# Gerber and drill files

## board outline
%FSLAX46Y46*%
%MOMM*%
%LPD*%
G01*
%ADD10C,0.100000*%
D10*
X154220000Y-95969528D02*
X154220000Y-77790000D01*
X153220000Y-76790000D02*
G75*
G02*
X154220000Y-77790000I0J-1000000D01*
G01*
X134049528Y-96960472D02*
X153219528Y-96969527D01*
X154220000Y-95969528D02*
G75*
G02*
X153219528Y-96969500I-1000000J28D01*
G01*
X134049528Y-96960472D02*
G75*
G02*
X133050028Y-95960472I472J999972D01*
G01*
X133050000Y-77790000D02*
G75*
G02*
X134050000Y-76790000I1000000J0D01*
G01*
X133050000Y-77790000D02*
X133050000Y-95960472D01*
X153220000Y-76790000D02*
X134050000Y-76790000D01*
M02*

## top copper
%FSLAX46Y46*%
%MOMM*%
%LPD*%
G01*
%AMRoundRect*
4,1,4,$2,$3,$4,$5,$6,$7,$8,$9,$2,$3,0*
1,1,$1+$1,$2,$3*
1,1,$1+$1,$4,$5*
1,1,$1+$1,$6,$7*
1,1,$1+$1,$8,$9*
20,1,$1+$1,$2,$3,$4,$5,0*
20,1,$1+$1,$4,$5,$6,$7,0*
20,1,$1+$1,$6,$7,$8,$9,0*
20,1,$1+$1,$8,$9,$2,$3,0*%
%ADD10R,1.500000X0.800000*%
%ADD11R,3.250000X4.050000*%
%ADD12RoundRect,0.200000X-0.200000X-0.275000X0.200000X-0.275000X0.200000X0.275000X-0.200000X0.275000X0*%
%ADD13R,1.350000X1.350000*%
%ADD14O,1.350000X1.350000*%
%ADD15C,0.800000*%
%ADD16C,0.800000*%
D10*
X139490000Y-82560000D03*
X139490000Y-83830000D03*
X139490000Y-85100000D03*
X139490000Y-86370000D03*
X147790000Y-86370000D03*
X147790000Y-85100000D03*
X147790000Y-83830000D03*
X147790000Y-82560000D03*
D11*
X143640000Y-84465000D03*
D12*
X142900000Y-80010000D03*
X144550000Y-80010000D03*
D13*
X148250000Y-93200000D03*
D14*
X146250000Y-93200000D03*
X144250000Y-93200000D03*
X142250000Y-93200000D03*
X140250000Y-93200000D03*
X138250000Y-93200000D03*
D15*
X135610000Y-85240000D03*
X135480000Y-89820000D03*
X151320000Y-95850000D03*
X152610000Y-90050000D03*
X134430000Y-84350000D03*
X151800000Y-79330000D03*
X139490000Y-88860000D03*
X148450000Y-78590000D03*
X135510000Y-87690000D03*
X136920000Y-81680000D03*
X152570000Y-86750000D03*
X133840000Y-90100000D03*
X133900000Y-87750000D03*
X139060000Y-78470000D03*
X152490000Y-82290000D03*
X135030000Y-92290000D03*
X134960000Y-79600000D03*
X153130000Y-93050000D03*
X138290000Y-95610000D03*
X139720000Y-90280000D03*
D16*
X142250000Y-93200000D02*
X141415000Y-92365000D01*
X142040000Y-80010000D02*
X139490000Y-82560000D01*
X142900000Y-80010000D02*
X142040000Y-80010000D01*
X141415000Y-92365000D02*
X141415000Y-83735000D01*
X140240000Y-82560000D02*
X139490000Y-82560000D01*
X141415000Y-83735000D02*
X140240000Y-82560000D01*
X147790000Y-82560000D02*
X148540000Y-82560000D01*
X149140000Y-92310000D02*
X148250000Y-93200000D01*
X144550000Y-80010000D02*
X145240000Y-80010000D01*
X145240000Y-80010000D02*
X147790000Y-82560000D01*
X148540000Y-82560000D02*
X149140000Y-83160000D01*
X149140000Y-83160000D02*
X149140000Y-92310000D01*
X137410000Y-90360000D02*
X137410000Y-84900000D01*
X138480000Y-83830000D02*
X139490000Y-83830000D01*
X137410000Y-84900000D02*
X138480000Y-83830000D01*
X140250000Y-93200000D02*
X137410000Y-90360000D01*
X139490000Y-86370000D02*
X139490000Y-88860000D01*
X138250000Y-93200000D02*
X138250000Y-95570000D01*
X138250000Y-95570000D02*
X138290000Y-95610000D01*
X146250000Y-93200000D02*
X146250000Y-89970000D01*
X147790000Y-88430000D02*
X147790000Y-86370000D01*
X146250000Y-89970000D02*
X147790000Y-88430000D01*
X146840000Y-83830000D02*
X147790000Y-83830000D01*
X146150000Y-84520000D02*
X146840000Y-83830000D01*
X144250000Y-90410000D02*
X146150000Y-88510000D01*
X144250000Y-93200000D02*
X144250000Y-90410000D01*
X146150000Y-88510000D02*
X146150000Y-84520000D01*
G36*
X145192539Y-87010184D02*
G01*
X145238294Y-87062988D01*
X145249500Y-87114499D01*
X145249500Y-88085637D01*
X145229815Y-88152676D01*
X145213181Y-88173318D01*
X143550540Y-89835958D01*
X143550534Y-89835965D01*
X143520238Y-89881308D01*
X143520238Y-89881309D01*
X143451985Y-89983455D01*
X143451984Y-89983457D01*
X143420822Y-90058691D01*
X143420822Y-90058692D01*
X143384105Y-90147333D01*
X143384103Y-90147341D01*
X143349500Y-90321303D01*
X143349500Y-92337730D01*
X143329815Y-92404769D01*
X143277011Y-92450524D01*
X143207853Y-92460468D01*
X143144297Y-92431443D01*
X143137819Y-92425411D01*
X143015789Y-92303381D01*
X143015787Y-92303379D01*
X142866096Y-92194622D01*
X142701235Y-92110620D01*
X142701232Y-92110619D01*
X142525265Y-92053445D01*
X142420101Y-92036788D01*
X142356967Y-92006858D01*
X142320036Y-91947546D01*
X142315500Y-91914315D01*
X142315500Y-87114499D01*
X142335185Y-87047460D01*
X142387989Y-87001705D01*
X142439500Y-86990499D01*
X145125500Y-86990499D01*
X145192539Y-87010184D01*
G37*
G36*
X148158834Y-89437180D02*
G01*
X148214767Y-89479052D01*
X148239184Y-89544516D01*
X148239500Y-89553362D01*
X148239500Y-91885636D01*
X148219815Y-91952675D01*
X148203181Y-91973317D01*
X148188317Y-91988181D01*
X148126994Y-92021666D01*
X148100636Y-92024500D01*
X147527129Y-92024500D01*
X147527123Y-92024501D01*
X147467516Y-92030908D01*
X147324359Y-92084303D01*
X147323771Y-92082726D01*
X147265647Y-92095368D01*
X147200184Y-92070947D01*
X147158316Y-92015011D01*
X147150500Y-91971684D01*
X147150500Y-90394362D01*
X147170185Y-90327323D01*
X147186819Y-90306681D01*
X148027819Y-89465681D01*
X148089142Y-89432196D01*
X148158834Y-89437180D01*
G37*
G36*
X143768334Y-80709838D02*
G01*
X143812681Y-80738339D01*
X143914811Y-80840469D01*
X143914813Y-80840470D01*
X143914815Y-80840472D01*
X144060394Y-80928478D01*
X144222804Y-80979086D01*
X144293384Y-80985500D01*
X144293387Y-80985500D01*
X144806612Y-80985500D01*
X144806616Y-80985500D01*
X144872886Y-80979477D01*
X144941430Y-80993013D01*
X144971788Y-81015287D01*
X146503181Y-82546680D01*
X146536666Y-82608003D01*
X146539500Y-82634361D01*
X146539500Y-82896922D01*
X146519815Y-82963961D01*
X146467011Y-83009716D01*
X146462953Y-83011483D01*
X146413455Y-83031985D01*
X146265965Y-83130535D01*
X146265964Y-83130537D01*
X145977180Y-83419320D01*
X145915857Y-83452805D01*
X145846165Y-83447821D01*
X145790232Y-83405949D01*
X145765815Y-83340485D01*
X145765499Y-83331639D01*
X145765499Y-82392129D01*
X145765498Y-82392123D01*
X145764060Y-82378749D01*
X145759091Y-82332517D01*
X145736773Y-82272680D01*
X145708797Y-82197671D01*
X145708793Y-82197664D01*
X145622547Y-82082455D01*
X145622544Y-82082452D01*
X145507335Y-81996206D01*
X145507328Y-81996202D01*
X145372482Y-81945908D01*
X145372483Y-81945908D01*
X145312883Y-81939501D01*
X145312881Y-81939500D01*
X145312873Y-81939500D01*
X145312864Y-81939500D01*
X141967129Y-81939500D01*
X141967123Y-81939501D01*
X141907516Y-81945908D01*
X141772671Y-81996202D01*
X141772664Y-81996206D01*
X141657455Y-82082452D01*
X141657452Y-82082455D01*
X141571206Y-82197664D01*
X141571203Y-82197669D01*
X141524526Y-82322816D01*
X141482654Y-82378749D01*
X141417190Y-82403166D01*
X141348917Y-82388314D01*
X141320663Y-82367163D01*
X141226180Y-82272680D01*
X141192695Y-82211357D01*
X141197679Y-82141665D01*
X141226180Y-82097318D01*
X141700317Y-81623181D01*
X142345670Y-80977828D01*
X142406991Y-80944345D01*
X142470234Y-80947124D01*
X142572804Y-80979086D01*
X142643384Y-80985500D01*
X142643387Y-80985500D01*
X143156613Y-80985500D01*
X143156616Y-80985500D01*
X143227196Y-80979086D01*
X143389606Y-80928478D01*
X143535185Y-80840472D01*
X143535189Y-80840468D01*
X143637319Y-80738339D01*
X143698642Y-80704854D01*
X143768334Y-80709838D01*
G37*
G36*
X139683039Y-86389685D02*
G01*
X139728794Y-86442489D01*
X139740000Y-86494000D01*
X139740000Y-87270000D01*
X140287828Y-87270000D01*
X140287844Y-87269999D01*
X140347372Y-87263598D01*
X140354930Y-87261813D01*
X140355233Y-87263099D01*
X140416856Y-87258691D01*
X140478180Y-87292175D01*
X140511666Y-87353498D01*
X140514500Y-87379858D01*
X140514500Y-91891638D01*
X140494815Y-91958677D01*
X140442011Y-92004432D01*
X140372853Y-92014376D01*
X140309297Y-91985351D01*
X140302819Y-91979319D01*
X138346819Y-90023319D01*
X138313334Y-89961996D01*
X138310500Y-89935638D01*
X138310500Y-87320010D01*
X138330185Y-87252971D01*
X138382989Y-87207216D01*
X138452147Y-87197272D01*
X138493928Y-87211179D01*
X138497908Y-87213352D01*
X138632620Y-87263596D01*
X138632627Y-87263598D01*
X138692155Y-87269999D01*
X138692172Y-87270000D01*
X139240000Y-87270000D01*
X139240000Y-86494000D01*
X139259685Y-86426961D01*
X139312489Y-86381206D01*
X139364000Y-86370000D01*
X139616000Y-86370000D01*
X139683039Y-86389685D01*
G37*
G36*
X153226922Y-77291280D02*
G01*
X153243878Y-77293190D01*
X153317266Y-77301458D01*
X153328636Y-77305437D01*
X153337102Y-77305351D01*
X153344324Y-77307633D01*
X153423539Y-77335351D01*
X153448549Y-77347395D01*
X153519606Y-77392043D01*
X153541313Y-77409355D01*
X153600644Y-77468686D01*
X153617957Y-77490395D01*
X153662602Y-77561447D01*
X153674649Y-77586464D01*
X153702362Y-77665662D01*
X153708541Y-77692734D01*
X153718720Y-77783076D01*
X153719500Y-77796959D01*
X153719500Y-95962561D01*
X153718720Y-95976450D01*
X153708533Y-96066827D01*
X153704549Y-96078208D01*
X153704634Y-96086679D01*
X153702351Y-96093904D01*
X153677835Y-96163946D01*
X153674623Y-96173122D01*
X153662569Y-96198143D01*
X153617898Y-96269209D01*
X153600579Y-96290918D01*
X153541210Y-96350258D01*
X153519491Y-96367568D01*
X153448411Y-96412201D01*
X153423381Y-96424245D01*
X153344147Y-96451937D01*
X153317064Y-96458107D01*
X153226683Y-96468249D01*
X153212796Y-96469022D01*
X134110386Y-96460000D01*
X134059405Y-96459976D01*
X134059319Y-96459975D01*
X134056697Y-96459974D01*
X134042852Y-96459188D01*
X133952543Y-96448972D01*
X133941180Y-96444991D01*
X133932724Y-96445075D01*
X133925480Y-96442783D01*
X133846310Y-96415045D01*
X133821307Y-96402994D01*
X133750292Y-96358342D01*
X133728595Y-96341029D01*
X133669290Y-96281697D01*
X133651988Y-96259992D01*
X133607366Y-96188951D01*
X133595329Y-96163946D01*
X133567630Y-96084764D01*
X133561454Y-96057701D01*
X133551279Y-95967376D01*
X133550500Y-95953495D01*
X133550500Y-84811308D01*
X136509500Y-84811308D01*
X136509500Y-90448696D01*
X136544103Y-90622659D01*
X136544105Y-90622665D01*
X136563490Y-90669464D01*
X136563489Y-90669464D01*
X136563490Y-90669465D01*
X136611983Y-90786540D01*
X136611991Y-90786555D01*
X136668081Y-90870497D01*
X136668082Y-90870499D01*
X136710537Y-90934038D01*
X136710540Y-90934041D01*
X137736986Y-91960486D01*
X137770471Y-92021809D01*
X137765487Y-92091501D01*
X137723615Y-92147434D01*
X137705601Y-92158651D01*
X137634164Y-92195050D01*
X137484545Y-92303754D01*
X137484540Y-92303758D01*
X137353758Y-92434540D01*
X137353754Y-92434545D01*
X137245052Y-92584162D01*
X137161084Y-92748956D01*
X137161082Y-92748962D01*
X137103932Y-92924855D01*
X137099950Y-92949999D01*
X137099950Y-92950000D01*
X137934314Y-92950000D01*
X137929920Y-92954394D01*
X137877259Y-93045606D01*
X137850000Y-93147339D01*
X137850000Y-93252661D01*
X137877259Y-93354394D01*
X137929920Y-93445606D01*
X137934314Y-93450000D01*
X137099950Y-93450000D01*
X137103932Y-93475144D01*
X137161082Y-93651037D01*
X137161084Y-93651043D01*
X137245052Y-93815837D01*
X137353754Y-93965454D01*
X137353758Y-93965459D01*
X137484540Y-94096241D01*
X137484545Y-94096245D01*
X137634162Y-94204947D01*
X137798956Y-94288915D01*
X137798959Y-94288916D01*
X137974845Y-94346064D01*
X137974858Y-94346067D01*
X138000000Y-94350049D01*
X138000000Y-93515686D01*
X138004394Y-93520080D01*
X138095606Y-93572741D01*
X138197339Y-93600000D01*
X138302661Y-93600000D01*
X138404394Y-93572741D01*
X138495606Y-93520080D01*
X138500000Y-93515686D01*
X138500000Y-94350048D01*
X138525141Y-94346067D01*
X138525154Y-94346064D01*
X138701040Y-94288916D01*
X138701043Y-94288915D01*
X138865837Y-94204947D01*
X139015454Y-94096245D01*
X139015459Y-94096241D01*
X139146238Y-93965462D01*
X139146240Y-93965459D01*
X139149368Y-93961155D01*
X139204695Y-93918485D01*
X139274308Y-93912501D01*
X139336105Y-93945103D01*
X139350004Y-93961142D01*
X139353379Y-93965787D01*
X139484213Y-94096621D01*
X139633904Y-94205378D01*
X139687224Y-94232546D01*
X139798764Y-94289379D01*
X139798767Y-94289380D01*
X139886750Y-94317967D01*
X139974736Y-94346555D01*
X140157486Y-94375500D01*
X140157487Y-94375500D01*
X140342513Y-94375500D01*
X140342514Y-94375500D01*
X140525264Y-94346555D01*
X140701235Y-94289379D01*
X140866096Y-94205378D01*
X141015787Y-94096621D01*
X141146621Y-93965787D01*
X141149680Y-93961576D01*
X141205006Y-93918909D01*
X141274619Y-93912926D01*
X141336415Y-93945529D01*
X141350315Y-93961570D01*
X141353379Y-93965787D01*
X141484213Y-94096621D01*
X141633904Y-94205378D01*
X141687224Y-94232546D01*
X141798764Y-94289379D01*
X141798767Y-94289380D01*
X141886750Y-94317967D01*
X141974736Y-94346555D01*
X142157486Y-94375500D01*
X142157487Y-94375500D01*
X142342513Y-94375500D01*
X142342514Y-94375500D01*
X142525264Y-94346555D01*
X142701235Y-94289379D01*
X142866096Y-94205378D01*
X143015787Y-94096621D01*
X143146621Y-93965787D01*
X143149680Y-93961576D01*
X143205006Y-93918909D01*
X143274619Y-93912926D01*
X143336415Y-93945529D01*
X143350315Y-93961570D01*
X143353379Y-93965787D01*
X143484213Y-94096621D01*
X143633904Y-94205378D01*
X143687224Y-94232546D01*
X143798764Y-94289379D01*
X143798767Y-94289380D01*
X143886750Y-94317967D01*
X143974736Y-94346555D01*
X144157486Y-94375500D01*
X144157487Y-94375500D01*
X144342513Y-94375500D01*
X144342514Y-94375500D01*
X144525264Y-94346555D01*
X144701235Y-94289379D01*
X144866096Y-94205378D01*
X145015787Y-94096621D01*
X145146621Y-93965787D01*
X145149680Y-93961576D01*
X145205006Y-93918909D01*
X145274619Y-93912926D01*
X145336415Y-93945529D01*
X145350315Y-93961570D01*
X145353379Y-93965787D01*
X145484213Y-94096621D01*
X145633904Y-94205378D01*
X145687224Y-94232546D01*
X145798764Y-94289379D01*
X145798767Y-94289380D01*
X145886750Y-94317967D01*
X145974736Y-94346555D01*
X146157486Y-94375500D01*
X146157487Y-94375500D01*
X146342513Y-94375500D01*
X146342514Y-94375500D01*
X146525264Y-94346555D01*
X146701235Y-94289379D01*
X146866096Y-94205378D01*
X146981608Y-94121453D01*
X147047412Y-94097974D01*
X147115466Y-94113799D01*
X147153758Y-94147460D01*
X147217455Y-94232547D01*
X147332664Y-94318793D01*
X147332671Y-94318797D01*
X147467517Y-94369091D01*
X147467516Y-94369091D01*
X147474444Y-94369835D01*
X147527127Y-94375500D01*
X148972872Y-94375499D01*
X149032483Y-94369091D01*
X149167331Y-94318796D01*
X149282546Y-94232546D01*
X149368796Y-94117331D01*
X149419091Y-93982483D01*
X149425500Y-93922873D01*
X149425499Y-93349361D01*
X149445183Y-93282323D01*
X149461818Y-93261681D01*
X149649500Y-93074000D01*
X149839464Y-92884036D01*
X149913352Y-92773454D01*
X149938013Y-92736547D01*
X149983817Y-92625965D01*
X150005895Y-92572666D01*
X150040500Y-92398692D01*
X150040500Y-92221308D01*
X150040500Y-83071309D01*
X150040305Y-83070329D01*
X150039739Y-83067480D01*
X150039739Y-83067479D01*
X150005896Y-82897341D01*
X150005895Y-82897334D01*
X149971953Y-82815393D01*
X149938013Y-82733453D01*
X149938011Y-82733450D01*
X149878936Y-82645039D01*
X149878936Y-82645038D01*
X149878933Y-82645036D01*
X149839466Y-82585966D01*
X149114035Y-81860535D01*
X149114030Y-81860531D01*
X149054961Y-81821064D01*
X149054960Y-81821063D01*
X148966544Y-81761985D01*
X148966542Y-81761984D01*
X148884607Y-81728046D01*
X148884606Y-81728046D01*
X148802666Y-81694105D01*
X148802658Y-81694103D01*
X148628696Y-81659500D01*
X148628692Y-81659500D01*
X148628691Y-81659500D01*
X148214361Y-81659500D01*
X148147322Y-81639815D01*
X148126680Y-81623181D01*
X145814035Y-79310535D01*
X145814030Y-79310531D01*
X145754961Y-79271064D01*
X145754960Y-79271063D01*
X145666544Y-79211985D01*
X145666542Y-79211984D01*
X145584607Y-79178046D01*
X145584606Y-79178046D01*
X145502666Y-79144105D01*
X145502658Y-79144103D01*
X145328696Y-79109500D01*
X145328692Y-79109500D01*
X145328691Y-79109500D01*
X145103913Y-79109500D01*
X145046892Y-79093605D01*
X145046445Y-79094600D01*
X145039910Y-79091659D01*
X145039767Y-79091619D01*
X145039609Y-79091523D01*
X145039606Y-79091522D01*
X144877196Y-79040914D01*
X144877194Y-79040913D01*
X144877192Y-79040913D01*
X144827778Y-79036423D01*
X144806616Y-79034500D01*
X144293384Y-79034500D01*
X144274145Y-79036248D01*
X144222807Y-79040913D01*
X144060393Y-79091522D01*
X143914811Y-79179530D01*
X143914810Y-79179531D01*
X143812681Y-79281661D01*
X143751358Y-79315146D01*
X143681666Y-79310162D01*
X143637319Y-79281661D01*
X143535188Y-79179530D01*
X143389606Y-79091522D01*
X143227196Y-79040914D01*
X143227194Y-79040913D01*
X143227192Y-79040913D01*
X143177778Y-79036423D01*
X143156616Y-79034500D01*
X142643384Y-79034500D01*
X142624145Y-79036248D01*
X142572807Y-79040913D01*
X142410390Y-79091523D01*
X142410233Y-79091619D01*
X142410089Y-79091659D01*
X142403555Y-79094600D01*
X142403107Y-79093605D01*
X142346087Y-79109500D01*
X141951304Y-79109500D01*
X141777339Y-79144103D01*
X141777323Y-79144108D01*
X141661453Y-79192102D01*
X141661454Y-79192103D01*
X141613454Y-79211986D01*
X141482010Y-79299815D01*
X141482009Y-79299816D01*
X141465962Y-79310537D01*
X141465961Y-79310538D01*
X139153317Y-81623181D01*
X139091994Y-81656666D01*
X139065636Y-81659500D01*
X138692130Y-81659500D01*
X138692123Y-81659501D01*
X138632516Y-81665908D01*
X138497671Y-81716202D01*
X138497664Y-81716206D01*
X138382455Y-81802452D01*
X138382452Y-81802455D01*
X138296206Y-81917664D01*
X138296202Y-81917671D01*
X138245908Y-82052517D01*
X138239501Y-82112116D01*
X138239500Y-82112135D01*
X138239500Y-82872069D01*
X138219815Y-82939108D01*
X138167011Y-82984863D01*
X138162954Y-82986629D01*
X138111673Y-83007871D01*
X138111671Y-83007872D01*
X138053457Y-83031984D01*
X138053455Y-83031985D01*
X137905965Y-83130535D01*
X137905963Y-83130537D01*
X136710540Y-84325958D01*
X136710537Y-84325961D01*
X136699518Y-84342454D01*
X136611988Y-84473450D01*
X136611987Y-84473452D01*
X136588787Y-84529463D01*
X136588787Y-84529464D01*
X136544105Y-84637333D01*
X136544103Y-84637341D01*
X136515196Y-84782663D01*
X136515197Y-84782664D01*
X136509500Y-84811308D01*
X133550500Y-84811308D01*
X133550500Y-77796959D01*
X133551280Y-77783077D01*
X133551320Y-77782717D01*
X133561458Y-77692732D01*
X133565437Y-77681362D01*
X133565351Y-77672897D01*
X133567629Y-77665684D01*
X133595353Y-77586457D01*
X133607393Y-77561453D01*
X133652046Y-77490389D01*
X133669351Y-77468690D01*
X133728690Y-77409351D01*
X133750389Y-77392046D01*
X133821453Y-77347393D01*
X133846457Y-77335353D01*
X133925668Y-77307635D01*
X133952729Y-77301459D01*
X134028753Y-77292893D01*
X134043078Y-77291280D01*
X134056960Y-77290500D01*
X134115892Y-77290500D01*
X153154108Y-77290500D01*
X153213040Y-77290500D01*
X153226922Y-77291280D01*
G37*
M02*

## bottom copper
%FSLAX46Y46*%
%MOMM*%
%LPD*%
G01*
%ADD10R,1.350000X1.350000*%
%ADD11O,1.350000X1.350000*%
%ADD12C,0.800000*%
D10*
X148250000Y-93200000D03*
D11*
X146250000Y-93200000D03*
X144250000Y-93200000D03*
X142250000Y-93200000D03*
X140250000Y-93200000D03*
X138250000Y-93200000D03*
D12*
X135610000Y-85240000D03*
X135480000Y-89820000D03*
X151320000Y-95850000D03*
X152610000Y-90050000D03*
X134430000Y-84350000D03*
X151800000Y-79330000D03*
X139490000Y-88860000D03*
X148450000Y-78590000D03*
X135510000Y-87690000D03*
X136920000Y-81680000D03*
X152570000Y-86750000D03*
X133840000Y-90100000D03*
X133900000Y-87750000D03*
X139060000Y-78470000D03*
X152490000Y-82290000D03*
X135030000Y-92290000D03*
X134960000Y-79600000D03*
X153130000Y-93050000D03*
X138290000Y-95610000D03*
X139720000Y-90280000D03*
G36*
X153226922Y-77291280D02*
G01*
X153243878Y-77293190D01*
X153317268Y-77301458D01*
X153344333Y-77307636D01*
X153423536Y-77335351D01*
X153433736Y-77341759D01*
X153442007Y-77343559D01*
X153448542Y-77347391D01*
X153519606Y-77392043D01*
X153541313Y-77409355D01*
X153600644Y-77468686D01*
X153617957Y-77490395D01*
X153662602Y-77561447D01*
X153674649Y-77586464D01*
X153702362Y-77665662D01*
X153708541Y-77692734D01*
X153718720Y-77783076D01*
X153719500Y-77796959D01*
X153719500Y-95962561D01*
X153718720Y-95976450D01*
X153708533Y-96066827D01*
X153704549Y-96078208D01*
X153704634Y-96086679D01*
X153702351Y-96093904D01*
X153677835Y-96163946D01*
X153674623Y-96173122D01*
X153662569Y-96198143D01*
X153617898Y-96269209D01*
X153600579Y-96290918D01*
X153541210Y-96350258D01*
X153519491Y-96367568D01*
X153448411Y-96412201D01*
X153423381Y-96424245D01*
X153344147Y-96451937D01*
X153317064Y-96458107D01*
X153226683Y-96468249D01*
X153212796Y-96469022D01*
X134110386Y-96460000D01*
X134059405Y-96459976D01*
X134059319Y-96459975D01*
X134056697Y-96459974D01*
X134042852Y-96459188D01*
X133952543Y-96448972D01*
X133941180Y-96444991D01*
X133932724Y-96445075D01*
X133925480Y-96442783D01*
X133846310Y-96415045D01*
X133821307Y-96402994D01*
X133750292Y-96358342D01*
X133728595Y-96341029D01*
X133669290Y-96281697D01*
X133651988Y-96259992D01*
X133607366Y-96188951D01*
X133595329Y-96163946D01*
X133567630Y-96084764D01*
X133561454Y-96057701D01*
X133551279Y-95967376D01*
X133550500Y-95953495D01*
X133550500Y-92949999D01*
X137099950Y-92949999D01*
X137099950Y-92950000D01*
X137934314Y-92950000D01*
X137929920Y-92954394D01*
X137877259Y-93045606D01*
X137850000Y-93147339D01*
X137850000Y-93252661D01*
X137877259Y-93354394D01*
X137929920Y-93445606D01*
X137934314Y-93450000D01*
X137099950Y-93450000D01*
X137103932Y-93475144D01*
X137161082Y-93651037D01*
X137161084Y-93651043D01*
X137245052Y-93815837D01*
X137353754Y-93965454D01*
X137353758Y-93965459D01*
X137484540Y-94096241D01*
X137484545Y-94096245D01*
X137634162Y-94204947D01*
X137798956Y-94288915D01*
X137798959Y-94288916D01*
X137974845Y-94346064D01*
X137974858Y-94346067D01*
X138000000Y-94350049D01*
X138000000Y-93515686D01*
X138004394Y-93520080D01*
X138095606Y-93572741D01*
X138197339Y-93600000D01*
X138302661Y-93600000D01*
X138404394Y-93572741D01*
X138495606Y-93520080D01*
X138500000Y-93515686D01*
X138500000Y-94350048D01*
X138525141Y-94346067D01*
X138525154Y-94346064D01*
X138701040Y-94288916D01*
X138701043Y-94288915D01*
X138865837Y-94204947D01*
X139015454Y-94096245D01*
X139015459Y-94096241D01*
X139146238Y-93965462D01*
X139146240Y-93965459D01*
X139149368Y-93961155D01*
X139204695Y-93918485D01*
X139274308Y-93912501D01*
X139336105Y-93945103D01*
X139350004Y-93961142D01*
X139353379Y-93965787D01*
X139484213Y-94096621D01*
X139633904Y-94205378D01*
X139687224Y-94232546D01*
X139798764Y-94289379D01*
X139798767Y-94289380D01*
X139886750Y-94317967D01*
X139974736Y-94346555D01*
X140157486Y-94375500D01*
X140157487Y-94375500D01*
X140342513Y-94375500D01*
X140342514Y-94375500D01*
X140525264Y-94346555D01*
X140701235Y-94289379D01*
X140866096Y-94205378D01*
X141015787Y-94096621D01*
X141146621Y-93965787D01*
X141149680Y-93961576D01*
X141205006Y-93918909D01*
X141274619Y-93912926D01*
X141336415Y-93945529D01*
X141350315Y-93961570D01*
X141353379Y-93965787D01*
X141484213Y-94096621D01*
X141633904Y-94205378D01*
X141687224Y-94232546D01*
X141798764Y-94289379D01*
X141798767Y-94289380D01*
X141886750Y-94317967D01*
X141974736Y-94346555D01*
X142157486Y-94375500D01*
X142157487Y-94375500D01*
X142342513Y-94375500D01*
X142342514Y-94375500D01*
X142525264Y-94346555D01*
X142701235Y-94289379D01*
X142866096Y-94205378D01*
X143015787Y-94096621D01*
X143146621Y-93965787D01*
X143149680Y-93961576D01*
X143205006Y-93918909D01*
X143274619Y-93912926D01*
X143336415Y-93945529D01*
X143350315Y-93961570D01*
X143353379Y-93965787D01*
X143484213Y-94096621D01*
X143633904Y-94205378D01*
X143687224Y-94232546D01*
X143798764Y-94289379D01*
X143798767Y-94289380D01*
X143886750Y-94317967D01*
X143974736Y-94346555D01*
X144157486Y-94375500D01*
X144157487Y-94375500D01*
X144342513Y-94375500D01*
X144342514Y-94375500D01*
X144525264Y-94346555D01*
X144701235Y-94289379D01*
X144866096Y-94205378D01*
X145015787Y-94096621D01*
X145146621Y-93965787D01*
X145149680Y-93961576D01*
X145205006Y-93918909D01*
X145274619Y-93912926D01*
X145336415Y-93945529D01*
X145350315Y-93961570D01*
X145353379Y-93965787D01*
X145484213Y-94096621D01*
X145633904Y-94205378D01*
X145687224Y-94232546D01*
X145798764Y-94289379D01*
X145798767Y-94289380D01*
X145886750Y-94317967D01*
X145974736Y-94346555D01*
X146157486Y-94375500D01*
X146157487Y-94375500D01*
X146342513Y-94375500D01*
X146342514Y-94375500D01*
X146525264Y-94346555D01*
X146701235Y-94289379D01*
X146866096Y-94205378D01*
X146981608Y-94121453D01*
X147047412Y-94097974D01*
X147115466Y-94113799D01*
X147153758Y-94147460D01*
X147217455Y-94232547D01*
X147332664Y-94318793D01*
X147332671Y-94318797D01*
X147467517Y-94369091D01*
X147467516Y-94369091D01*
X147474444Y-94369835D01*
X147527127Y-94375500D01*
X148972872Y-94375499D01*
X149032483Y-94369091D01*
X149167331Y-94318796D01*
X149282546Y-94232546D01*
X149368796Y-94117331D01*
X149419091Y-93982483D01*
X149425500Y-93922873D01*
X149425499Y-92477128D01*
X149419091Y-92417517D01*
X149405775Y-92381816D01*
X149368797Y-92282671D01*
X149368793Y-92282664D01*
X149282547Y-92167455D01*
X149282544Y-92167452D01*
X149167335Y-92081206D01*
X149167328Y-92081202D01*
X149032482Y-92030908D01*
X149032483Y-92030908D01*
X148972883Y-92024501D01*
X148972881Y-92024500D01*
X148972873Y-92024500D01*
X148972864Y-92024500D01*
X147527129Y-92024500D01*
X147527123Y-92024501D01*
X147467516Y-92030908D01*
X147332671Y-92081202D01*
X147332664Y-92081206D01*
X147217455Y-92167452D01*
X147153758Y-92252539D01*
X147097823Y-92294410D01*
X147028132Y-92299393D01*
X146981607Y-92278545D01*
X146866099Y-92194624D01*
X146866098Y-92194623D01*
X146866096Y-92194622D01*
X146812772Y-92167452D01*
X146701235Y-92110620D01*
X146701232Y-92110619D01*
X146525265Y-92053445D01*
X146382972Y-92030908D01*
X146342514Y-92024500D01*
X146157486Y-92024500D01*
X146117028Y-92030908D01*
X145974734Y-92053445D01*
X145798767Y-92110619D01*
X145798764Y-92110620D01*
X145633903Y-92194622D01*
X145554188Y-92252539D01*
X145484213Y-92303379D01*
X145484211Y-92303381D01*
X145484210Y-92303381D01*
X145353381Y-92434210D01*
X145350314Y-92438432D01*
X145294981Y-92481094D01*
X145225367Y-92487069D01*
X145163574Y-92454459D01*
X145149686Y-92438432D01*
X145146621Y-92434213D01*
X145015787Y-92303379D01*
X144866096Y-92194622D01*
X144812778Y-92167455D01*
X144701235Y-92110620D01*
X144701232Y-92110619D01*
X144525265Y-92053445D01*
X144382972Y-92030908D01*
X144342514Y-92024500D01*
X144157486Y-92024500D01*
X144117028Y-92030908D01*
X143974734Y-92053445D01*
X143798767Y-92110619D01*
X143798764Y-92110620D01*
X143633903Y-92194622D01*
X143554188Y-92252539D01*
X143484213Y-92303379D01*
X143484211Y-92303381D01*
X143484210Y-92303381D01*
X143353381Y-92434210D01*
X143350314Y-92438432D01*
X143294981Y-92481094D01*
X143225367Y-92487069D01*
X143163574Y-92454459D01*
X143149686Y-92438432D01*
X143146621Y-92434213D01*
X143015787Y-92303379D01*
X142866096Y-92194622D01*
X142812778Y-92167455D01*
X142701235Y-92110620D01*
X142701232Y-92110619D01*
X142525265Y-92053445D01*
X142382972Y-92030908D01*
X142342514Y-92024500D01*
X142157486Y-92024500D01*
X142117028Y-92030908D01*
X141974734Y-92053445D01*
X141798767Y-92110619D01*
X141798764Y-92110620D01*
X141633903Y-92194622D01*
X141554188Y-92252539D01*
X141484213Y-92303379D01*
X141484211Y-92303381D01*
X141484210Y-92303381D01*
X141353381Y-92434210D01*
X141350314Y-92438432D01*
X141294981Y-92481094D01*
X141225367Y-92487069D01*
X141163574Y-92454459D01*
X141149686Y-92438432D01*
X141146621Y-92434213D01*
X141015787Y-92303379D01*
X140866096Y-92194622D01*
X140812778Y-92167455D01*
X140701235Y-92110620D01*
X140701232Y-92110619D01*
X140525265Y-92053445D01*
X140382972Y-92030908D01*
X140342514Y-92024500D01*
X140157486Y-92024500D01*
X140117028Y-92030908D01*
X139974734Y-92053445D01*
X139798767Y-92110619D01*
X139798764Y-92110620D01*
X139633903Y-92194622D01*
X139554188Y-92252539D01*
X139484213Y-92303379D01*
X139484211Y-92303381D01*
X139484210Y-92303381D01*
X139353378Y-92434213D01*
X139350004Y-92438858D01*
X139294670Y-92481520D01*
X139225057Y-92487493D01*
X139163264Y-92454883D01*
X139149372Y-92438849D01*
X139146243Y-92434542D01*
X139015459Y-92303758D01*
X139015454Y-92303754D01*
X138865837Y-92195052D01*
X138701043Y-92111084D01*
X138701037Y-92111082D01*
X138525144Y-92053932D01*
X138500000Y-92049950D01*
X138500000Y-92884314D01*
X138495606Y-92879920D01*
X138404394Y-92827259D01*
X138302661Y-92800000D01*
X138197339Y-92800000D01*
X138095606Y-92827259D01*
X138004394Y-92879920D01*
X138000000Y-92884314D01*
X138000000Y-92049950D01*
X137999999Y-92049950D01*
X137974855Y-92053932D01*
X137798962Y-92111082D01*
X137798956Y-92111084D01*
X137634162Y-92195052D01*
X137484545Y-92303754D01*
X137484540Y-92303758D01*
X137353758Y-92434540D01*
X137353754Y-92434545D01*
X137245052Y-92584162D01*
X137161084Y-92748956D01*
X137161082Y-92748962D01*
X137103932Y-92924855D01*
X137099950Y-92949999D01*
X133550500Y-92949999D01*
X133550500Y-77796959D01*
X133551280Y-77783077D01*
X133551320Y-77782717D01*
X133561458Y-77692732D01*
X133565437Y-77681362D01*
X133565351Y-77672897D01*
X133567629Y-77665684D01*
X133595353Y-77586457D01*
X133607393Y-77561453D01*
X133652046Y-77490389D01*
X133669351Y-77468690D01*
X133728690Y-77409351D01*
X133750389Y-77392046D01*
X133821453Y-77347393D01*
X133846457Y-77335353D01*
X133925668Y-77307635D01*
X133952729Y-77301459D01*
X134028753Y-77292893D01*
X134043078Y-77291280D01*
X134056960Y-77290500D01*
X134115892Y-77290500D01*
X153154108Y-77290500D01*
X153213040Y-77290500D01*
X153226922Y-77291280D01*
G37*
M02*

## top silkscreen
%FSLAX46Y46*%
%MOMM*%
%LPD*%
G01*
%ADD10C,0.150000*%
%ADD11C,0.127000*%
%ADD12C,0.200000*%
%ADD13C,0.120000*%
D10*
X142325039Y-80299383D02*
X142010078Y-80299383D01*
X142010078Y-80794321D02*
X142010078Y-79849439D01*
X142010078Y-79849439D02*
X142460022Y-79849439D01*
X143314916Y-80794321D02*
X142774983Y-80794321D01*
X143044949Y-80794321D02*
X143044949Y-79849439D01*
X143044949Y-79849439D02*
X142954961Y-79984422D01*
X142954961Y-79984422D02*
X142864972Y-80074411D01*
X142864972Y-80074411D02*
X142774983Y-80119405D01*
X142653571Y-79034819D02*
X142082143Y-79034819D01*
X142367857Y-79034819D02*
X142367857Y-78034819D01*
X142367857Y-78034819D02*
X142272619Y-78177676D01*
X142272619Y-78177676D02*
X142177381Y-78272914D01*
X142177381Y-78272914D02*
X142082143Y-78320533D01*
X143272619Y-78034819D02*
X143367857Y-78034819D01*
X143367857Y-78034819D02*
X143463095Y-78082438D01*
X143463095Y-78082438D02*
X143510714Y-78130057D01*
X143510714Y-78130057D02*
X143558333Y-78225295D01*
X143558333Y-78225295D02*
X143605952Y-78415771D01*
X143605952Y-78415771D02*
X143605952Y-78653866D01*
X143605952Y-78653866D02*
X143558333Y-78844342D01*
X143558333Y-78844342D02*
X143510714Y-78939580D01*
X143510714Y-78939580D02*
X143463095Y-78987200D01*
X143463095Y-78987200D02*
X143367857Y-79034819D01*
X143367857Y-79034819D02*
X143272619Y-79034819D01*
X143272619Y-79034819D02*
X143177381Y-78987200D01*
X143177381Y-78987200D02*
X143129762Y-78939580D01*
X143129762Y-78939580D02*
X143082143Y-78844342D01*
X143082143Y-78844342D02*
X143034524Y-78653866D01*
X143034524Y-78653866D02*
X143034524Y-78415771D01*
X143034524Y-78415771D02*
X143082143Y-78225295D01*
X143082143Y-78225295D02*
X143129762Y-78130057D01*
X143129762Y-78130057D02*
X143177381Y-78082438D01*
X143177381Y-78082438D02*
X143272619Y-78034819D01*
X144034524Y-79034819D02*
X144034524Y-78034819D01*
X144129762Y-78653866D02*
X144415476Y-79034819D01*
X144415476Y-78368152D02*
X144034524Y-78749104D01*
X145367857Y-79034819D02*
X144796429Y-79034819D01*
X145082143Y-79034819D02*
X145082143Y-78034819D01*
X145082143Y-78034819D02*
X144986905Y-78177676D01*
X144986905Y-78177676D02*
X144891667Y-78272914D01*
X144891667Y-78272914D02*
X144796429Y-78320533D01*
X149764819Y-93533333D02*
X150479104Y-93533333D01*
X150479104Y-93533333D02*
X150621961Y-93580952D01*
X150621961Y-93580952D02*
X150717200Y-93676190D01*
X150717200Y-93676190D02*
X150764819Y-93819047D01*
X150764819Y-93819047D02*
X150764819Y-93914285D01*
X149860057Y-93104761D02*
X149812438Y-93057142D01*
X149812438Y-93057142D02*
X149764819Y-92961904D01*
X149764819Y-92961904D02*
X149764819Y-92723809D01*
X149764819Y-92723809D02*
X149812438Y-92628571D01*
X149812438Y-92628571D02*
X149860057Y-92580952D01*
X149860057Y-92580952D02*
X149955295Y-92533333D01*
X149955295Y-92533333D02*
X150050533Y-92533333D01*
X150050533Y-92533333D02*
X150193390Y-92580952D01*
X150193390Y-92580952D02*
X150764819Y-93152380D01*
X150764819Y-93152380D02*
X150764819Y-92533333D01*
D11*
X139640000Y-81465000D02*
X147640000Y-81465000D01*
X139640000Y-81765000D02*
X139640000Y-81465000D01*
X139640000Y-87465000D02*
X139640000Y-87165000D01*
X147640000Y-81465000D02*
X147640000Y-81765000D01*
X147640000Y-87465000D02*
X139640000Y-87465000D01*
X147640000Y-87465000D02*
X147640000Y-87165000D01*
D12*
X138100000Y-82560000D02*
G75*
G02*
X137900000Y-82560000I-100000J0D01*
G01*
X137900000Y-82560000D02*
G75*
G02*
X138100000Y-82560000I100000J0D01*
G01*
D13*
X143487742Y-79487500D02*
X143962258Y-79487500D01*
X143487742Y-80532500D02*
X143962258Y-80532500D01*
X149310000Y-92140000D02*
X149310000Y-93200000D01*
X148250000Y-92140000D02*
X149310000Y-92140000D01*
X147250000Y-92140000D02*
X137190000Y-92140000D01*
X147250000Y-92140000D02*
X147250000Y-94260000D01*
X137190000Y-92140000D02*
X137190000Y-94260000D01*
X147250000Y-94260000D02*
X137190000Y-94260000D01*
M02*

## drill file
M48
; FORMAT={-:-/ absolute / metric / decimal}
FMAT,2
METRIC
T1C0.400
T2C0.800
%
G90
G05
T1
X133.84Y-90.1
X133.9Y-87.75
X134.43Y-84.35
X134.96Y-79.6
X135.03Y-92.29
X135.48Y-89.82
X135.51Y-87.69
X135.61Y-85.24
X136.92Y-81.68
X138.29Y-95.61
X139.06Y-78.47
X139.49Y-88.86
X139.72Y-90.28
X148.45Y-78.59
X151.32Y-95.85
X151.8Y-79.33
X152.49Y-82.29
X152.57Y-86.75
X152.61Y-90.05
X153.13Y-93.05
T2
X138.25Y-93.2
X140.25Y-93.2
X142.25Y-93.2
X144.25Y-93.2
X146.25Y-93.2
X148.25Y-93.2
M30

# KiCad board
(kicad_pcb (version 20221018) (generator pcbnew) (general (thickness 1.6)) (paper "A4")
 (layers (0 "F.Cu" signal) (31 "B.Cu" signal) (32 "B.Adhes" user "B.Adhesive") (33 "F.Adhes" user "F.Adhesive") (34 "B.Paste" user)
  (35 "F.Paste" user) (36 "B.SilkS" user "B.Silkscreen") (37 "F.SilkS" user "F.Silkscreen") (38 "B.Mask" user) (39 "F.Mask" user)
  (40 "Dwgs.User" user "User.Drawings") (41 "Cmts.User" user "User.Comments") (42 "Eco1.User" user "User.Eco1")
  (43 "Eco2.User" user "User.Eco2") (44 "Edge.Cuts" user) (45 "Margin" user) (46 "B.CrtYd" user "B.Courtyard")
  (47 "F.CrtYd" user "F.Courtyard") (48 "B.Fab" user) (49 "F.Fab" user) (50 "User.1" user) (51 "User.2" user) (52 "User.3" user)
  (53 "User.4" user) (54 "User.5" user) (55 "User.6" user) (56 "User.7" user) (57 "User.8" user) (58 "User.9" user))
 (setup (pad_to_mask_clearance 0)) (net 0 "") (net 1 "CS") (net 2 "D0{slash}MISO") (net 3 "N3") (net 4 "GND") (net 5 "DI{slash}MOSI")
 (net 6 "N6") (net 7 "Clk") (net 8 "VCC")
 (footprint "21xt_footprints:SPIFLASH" (layer "F.Cu") (at 143.64 84.465)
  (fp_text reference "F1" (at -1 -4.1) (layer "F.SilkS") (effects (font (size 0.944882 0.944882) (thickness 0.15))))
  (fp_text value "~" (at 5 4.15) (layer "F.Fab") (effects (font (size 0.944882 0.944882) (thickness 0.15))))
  (fp_line (start -4 -3) (end 4 -3) (stroke (width 0.127) (type solid)) (layer "F.SilkS"))
  (fp_line (start -4 -2.7) (end -4 -3) (stroke (width 0.127) (type solid)) (layer "F.SilkS"))
  (fp_line (start -4 3) (end -4 2.7) (stroke (width 0.127) (type solid)) (layer "F.SilkS"))
  (fp_line (start 4 -3) (end 4 -2.7) (stroke (width 0.127) (type solid)) (layer "F.SilkS"))
  (fp_line (start 4 3) (end -4 3) (stroke (width 0.127) (type solid)) (layer "F.SilkS"))
  (fp_line (start 4 3) (end 4 2.7) (stroke (width 0.127) (type solid)) (layer "F.SilkS"))
  (fp_circle (center -5.64 -1.905) (end -5.54 -1.905) (stroke (width 0.2) (type solid)) (fill none) (layer "F.SilkS"))
  (pad "1" smd rect (at -4.15 -1.905) (size 1.5 0.8) (layers "F.Cu" "F.Mask") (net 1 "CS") (solder_mask_margin 0.102))
  (pad "2" smd rect (at -4.15 -0.635) (size 1.5 0.8) (layers "F.Cu" "F.Mask") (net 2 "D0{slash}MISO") (solder_mask_margin 0.102))
  (pad "3" smd rect (at -4.15 0.635) (size 1.5 0.8) (layers "F.Cu" "F.Mask") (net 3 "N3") (solder_mask_margin 0.102))
  (pad "4" smd rect (at -4.15 1.905) (size 1.5 0.8) (layers "F.Cu" "F.Mask") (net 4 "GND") (solder_mask_margin 0.102))
  (pad "5" smd rect (at 4.15 1.905) (size 1.5 0.8) (layers "F.Cu" "F.Mask") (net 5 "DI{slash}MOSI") (solder_mask_margin 0.102))
  (pad "6" smd rect (at 4.15 0.635) (size 1.5 0.8) (layers "F.Cu" "F.Mask") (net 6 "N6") (solder_mask_margin 0.102))
  (pad "7" smd rect (at 4.15 -0.635) (size 1.5 0.8) (layers "F.Cu" "F.Mask") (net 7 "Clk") (solder_mask_margin 0.102))
  (pad "8" smd rect (at 4.15 -1.905) (size 1.5 0.8) (layers "F.Cu" "F.Mask") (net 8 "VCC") (solder_mask_margin 0.102))
  (pad "9" smd rect (at 0 0) (size 3.25 4.05) (layers "F.Cu" "F.Mask") (solder_mask_margin 0.102)))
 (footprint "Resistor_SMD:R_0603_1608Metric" (layer "F.Cu") (at 143.725 80.01)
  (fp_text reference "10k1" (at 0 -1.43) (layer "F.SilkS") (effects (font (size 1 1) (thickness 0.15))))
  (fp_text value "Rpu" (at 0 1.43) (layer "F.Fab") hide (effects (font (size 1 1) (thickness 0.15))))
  (fp_line (start -0.237258 -0.5225) (end 0.237258 -0.5225) (stroke (width 0.12) (type solid)) (layer "F.SilkS"))
  (fp_line (start -0.237258 0.5225) (end 0.237258 0.5225) (stroke (width 0.12) (type solid)) (layer "F.SilkS"))
  (pad "1" smd roundrect (at -0.825 0) (size 0.8 0.95) (layers "F.Cu" "F.Paste" "F.Mask") (roundrect_rratio 0.25) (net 1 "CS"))
  (pad "2" smd roundrect (at 0.825 0) (size 0.8 0.95) (layers "F.Cu" "F.Paste" "F.Mask") (roundrect_rratio 0.25) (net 8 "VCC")))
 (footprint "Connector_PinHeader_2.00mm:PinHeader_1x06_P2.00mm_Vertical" (layer "F.Cu") (at 148.25 93.2 -90)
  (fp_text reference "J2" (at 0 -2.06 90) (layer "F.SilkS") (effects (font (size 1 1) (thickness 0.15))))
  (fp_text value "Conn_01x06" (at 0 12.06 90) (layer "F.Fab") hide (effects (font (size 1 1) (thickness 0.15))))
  (fp_line (start -1.06 -1.06) (end 0 -1.06) (stroke (width 0.12) (type solid)) (layer "F.SilkS"))
  (fp_line (start -1.06 0) (end -1.06 -1.06) (stroke (width 0.12) (type solid)) (layer "F.SilkS"))
  (fp_line (start -1.06 1) (end -1.06 11.06) (stroke (width 0.12) (type solid)) (layer "F.SilkS"))
  (fp_line (start -1.06 1) (end 1.06 1) (stroke (width 0.12) (type solid)) (layer "F.SilkS"))
  (fp_line (start -1.06 11.06) (end 1.06 11.06) (stroke (width 0.12) (type solid)) (layer "F.SilkS"))
  (fp_line (start 1.06 1) (end 1.06 11.06) (stroke (width 0.12) (type solid)) (layer "F.SilkS"))
  (pad "1" thru_hole rect (at 0 0 270) (size 1.35 1.35) (drill 0.8) (layers "*.Cu" "*.Mask") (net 8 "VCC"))
  (pad "2" thru_hole oval (at 0 2 270) (size 1.35 1.35) (drill 0.8) (layers "*.Cu" "*.Mask") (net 5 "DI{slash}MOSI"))
  (pad "3" thru_hole oval (at 0 4 270) (size 1.35 1.35) (drill 0.8) (layers "*.Cu" "*.Mask") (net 7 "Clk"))
  (pad "4" thru_hole oval (at 0 6 270) (size 1.35 1.35) (drill 0.8) (layers "*.Cu" "*.Mask") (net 1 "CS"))
  (pad "5" thru_hole oval (at 0 8 270) (size 1.35 1.35) (drill 0.8) (layers "*.Cu" "*.Mask") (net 2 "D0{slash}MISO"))
  (pad "6" thru_hole oval (at 0 10 270) (size 1.35 1.35) (drill 0.8) (layers "*.Cu" "*.Mask") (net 4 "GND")))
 (gr_line (start 154.22 95.969528) (end 154.22 77.79) (stroke (width 0.1) (type default)) (layer "Edge.Cuts"))
 (gr_arc (start 153.22 76.79) (mid 153.927107 77.082893) (end 154.22 77.79) (stroke (width 0.1) (type default)) (layer "Edge.Cuts"))
 (gr_line (start 134.049528 96.960472) (end 153.219528 96.969527) (stroke (width 0.1) (type default)) (layer "Edge.Cuts"))
 (gr_arc (start 154.22 95.969528) (mid 153.92694 96.676802) (end 153.219528 96.969527) (stroke (width 0.1) (type default))
  (layer "Edge.Cuts"))
 (gr_arc (start 134.049528 96.960472) (mid 133.342736 96.66741) (end 133.05 95.960472) (stroke (width 0.1) (type default))
  (layer "Edge.Cuts"))
 (gr_arc (start 133.05 77.79) (mid 133.342893 77.082893) (end 134.05 76.79) (stroke (width 0.1) (type default)) (layer "Edge.Cuts"))
 (gr_line (start 133.05 77.79) (end 133.05 95.960472) (stroke (width 0.1) (type default)) (layer "Edge.Cuts"))
 (gr_line (start 153.22 76.79) (end 134.05 76.79) (stroke (width 0.1) (type default)) (layer "Edge.Cuts"))
 (segment (start 142.25 93.2) (end 141.415 92.365) (width 0.8) (layer "F.Cu") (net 1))
 (segment (start 142.04 80.01) (end 139.49 82.56) (width 0.8) (layer "F.Cu") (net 1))
 (segment (start 142.9 80.01) (end 142.04 80.01) (width 0.8) (layer "F.Cu") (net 1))
 (segment (start 141.415 92.365) (end 141.415 83.735) (width 0.8) (layer "F.Cu") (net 1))
 (segment (start 140.24 82.56) (end 139.49 82.56) (width 0.8) (layer "F.Cu") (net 1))
 (segment (start 141.415 83.735) (end 140.24 82.56) (width 0.8) (layer "F.Cu") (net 1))
 (segment (start 147.79 82.56) (end 148.54 82.56) (width 0.8) (layer "F.Cu") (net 8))
 (segment (start 149.14 92.31) (end 148.25 93.2) (width 0.8) (layer "F.Cu") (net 8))
 (segment (start 144.55 80.01) (end 145.24 80.01) (width 0.8) (layer "F.Cu") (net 8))
 (segment (start 145.24 80.01) (end 147.79 82.56) (width 0.8) (layer "F.Cu") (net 8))
 (segment (start 148.54 82.56) (end 149.14 83.16) (width 0.8) (layer "F.Cu") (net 8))
 (segment (start 149.14 83.16) (end 149.14 92.31) (width 0.8) (layer "F.Cu") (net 8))
 (segment (start 137.41 90.36) (end 137.41 84.9) (width 0.8) (layer "F.Cu") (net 2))
 (segment (start 138.48 83.83) (end 139.49 83.83) (width 0.8) (layer "F.Cu") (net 2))
 (segment (start 137.41 84.9) (end 138.48 83.83) (width 0.8) (layer "F.Cu") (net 2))
 (segment (start 140.25 93.2) (end 137.41 90.36) (width 0.8) (layer "F.Cu") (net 2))
 (segment (start 139.49 86.37) (end 139.49 88.86) (width 0.8) (layer "F.Cu") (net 4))
 (segment (start 138.25 93.2) (end 138.25 95.57) (width 0.8) (layer "F.Cu") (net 4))
 (segment (start 138.25 95.57) (end 138.29 95.61) (width 0.8) (layer "F.Cu") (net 4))
 (via (at 135.61 85.24) (size 0.8) (drill 0.4) (layers "F.Cu" "B.Cu") (free) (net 4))
 (via (at 135.48 89.82) (size 0.8) (drill 0.4) (layers "F.Cu" "B.Cu") (free) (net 4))
 (via (at 151.32 95.85) (size 0.8) (drill 0.4) (layers "F.Cu" "B.Cu") (free) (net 4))
 (via (at 152.61 90.05) (size 0.8) (drill 0.4) (layers "F.Cu" "B.Cu") (free) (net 4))
 (via (at 134.43 84.35) (size 0.8) (drill 0.4) (layers "F.Cu" "B.Cu") (free) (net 4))
 (via (at 151.8 79.33) (size 0.8) (drill 0.4) (layers "F.Cu" "B.Cu") (free) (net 4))
 (via (at 139.49 88.86) (size 0.8) (drill 0.4) (layers "F.Cu" "B.Cu") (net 4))
 (via (at 148.45 78.59) (size 0.8) (drill 0.4) (layers "F.Cu" "B.Cu") (free) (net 4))
 (via (at 135.51 87.69) (size 0.8) (drill 0.4) (layers "F.Cu" "B.Cu") (free) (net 4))
 (via (at 136.92 81.68) (size 0.8) (drill 0.4) (layers "F.Cu" "B.Cu") (free) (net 4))
 (via (at 152.57 86.75) (size 0.8) (drill 0.4) (layers "F.Cu" "B.Cu") (free) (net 4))
 (via (at 133.84 90.1) (size 0.8) (drill 0.4) (layers "F.Cu" "B.Cu") (free) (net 4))
 (via (at 133.9 87.75) (size 0.8) (drill 0.4) (layers "F.Cu" "B.Cu") (free) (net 4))
 (via (at 139.06 78.47) (size 0.8) (drill 0.4) (layers "F.Cu" "B.Cu") (free) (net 4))
 (via (at 152.49 82.29) (size 0.8) (drill 0.4) (layers "F.Cu" "B.Cu") (free) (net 4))
 (via (at 135.03 92.29) (size 0.8) (drill 0.4) (layers "F.Cu" "B.Cu") (free) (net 4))
 (via (at 134.96 79.6) (size 0.8) (drill 0.4) (layers "F.Cu" "B.Cu") (free) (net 4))
 (via (at 153.13 93.05) (size 0.8) (drill 0.4) (layers "F.Cu" "B.Cu") (free) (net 4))
 (via (at 138.29 95.61) (size 0.8) (drill 0.4) (layers "F.Cu" "B.Cu") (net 4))
 (via (at 139.72 90.28) (size 0.8) (drill 0.4) (layers "F.Cu" "B.Cu") (free) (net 4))
 (segment (start 146.25 93.2) (end 146.25 89.97) (width 0.8) (layer "F.Cu") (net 5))
 (segment (start 147.79 88.43) (end 147.79 86.37) (width 0.8) (layer "F.Cu") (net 5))
 (segment (start 146.25 89.97) (end 147.79 88.43) (width 0.8) (layer "F.Cu") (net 5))
 (segment (start 146.84 83.83) (end 147.79 83.83) (width 0.8) (layer "F.Cu") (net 7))
 (segment (start 146.15 84.52) (end 146.84 83.83) (width 0.8) (layer "F.Cu") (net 7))
 (segment (start 144.25 90.41) (end 146.15 88.51) (width 0.8) (layer "F.Cu") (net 7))
 (segment (start 144.25 93.2) (end 144.25 90.41) (width 0.8) (layer "F.Cu") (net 7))
 (segment (start 146.15 88.51) (end 146.15 84.52) (width 0.8) (layer "F.Cu") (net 7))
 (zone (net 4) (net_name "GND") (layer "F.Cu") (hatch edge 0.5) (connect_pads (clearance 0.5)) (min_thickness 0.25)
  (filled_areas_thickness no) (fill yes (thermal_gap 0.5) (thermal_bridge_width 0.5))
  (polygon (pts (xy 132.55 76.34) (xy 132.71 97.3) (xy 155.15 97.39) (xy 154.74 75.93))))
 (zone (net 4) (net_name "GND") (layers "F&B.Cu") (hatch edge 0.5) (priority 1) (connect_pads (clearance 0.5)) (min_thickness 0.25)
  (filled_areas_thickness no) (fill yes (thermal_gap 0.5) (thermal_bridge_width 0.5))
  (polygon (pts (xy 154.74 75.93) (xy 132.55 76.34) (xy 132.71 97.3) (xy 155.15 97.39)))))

